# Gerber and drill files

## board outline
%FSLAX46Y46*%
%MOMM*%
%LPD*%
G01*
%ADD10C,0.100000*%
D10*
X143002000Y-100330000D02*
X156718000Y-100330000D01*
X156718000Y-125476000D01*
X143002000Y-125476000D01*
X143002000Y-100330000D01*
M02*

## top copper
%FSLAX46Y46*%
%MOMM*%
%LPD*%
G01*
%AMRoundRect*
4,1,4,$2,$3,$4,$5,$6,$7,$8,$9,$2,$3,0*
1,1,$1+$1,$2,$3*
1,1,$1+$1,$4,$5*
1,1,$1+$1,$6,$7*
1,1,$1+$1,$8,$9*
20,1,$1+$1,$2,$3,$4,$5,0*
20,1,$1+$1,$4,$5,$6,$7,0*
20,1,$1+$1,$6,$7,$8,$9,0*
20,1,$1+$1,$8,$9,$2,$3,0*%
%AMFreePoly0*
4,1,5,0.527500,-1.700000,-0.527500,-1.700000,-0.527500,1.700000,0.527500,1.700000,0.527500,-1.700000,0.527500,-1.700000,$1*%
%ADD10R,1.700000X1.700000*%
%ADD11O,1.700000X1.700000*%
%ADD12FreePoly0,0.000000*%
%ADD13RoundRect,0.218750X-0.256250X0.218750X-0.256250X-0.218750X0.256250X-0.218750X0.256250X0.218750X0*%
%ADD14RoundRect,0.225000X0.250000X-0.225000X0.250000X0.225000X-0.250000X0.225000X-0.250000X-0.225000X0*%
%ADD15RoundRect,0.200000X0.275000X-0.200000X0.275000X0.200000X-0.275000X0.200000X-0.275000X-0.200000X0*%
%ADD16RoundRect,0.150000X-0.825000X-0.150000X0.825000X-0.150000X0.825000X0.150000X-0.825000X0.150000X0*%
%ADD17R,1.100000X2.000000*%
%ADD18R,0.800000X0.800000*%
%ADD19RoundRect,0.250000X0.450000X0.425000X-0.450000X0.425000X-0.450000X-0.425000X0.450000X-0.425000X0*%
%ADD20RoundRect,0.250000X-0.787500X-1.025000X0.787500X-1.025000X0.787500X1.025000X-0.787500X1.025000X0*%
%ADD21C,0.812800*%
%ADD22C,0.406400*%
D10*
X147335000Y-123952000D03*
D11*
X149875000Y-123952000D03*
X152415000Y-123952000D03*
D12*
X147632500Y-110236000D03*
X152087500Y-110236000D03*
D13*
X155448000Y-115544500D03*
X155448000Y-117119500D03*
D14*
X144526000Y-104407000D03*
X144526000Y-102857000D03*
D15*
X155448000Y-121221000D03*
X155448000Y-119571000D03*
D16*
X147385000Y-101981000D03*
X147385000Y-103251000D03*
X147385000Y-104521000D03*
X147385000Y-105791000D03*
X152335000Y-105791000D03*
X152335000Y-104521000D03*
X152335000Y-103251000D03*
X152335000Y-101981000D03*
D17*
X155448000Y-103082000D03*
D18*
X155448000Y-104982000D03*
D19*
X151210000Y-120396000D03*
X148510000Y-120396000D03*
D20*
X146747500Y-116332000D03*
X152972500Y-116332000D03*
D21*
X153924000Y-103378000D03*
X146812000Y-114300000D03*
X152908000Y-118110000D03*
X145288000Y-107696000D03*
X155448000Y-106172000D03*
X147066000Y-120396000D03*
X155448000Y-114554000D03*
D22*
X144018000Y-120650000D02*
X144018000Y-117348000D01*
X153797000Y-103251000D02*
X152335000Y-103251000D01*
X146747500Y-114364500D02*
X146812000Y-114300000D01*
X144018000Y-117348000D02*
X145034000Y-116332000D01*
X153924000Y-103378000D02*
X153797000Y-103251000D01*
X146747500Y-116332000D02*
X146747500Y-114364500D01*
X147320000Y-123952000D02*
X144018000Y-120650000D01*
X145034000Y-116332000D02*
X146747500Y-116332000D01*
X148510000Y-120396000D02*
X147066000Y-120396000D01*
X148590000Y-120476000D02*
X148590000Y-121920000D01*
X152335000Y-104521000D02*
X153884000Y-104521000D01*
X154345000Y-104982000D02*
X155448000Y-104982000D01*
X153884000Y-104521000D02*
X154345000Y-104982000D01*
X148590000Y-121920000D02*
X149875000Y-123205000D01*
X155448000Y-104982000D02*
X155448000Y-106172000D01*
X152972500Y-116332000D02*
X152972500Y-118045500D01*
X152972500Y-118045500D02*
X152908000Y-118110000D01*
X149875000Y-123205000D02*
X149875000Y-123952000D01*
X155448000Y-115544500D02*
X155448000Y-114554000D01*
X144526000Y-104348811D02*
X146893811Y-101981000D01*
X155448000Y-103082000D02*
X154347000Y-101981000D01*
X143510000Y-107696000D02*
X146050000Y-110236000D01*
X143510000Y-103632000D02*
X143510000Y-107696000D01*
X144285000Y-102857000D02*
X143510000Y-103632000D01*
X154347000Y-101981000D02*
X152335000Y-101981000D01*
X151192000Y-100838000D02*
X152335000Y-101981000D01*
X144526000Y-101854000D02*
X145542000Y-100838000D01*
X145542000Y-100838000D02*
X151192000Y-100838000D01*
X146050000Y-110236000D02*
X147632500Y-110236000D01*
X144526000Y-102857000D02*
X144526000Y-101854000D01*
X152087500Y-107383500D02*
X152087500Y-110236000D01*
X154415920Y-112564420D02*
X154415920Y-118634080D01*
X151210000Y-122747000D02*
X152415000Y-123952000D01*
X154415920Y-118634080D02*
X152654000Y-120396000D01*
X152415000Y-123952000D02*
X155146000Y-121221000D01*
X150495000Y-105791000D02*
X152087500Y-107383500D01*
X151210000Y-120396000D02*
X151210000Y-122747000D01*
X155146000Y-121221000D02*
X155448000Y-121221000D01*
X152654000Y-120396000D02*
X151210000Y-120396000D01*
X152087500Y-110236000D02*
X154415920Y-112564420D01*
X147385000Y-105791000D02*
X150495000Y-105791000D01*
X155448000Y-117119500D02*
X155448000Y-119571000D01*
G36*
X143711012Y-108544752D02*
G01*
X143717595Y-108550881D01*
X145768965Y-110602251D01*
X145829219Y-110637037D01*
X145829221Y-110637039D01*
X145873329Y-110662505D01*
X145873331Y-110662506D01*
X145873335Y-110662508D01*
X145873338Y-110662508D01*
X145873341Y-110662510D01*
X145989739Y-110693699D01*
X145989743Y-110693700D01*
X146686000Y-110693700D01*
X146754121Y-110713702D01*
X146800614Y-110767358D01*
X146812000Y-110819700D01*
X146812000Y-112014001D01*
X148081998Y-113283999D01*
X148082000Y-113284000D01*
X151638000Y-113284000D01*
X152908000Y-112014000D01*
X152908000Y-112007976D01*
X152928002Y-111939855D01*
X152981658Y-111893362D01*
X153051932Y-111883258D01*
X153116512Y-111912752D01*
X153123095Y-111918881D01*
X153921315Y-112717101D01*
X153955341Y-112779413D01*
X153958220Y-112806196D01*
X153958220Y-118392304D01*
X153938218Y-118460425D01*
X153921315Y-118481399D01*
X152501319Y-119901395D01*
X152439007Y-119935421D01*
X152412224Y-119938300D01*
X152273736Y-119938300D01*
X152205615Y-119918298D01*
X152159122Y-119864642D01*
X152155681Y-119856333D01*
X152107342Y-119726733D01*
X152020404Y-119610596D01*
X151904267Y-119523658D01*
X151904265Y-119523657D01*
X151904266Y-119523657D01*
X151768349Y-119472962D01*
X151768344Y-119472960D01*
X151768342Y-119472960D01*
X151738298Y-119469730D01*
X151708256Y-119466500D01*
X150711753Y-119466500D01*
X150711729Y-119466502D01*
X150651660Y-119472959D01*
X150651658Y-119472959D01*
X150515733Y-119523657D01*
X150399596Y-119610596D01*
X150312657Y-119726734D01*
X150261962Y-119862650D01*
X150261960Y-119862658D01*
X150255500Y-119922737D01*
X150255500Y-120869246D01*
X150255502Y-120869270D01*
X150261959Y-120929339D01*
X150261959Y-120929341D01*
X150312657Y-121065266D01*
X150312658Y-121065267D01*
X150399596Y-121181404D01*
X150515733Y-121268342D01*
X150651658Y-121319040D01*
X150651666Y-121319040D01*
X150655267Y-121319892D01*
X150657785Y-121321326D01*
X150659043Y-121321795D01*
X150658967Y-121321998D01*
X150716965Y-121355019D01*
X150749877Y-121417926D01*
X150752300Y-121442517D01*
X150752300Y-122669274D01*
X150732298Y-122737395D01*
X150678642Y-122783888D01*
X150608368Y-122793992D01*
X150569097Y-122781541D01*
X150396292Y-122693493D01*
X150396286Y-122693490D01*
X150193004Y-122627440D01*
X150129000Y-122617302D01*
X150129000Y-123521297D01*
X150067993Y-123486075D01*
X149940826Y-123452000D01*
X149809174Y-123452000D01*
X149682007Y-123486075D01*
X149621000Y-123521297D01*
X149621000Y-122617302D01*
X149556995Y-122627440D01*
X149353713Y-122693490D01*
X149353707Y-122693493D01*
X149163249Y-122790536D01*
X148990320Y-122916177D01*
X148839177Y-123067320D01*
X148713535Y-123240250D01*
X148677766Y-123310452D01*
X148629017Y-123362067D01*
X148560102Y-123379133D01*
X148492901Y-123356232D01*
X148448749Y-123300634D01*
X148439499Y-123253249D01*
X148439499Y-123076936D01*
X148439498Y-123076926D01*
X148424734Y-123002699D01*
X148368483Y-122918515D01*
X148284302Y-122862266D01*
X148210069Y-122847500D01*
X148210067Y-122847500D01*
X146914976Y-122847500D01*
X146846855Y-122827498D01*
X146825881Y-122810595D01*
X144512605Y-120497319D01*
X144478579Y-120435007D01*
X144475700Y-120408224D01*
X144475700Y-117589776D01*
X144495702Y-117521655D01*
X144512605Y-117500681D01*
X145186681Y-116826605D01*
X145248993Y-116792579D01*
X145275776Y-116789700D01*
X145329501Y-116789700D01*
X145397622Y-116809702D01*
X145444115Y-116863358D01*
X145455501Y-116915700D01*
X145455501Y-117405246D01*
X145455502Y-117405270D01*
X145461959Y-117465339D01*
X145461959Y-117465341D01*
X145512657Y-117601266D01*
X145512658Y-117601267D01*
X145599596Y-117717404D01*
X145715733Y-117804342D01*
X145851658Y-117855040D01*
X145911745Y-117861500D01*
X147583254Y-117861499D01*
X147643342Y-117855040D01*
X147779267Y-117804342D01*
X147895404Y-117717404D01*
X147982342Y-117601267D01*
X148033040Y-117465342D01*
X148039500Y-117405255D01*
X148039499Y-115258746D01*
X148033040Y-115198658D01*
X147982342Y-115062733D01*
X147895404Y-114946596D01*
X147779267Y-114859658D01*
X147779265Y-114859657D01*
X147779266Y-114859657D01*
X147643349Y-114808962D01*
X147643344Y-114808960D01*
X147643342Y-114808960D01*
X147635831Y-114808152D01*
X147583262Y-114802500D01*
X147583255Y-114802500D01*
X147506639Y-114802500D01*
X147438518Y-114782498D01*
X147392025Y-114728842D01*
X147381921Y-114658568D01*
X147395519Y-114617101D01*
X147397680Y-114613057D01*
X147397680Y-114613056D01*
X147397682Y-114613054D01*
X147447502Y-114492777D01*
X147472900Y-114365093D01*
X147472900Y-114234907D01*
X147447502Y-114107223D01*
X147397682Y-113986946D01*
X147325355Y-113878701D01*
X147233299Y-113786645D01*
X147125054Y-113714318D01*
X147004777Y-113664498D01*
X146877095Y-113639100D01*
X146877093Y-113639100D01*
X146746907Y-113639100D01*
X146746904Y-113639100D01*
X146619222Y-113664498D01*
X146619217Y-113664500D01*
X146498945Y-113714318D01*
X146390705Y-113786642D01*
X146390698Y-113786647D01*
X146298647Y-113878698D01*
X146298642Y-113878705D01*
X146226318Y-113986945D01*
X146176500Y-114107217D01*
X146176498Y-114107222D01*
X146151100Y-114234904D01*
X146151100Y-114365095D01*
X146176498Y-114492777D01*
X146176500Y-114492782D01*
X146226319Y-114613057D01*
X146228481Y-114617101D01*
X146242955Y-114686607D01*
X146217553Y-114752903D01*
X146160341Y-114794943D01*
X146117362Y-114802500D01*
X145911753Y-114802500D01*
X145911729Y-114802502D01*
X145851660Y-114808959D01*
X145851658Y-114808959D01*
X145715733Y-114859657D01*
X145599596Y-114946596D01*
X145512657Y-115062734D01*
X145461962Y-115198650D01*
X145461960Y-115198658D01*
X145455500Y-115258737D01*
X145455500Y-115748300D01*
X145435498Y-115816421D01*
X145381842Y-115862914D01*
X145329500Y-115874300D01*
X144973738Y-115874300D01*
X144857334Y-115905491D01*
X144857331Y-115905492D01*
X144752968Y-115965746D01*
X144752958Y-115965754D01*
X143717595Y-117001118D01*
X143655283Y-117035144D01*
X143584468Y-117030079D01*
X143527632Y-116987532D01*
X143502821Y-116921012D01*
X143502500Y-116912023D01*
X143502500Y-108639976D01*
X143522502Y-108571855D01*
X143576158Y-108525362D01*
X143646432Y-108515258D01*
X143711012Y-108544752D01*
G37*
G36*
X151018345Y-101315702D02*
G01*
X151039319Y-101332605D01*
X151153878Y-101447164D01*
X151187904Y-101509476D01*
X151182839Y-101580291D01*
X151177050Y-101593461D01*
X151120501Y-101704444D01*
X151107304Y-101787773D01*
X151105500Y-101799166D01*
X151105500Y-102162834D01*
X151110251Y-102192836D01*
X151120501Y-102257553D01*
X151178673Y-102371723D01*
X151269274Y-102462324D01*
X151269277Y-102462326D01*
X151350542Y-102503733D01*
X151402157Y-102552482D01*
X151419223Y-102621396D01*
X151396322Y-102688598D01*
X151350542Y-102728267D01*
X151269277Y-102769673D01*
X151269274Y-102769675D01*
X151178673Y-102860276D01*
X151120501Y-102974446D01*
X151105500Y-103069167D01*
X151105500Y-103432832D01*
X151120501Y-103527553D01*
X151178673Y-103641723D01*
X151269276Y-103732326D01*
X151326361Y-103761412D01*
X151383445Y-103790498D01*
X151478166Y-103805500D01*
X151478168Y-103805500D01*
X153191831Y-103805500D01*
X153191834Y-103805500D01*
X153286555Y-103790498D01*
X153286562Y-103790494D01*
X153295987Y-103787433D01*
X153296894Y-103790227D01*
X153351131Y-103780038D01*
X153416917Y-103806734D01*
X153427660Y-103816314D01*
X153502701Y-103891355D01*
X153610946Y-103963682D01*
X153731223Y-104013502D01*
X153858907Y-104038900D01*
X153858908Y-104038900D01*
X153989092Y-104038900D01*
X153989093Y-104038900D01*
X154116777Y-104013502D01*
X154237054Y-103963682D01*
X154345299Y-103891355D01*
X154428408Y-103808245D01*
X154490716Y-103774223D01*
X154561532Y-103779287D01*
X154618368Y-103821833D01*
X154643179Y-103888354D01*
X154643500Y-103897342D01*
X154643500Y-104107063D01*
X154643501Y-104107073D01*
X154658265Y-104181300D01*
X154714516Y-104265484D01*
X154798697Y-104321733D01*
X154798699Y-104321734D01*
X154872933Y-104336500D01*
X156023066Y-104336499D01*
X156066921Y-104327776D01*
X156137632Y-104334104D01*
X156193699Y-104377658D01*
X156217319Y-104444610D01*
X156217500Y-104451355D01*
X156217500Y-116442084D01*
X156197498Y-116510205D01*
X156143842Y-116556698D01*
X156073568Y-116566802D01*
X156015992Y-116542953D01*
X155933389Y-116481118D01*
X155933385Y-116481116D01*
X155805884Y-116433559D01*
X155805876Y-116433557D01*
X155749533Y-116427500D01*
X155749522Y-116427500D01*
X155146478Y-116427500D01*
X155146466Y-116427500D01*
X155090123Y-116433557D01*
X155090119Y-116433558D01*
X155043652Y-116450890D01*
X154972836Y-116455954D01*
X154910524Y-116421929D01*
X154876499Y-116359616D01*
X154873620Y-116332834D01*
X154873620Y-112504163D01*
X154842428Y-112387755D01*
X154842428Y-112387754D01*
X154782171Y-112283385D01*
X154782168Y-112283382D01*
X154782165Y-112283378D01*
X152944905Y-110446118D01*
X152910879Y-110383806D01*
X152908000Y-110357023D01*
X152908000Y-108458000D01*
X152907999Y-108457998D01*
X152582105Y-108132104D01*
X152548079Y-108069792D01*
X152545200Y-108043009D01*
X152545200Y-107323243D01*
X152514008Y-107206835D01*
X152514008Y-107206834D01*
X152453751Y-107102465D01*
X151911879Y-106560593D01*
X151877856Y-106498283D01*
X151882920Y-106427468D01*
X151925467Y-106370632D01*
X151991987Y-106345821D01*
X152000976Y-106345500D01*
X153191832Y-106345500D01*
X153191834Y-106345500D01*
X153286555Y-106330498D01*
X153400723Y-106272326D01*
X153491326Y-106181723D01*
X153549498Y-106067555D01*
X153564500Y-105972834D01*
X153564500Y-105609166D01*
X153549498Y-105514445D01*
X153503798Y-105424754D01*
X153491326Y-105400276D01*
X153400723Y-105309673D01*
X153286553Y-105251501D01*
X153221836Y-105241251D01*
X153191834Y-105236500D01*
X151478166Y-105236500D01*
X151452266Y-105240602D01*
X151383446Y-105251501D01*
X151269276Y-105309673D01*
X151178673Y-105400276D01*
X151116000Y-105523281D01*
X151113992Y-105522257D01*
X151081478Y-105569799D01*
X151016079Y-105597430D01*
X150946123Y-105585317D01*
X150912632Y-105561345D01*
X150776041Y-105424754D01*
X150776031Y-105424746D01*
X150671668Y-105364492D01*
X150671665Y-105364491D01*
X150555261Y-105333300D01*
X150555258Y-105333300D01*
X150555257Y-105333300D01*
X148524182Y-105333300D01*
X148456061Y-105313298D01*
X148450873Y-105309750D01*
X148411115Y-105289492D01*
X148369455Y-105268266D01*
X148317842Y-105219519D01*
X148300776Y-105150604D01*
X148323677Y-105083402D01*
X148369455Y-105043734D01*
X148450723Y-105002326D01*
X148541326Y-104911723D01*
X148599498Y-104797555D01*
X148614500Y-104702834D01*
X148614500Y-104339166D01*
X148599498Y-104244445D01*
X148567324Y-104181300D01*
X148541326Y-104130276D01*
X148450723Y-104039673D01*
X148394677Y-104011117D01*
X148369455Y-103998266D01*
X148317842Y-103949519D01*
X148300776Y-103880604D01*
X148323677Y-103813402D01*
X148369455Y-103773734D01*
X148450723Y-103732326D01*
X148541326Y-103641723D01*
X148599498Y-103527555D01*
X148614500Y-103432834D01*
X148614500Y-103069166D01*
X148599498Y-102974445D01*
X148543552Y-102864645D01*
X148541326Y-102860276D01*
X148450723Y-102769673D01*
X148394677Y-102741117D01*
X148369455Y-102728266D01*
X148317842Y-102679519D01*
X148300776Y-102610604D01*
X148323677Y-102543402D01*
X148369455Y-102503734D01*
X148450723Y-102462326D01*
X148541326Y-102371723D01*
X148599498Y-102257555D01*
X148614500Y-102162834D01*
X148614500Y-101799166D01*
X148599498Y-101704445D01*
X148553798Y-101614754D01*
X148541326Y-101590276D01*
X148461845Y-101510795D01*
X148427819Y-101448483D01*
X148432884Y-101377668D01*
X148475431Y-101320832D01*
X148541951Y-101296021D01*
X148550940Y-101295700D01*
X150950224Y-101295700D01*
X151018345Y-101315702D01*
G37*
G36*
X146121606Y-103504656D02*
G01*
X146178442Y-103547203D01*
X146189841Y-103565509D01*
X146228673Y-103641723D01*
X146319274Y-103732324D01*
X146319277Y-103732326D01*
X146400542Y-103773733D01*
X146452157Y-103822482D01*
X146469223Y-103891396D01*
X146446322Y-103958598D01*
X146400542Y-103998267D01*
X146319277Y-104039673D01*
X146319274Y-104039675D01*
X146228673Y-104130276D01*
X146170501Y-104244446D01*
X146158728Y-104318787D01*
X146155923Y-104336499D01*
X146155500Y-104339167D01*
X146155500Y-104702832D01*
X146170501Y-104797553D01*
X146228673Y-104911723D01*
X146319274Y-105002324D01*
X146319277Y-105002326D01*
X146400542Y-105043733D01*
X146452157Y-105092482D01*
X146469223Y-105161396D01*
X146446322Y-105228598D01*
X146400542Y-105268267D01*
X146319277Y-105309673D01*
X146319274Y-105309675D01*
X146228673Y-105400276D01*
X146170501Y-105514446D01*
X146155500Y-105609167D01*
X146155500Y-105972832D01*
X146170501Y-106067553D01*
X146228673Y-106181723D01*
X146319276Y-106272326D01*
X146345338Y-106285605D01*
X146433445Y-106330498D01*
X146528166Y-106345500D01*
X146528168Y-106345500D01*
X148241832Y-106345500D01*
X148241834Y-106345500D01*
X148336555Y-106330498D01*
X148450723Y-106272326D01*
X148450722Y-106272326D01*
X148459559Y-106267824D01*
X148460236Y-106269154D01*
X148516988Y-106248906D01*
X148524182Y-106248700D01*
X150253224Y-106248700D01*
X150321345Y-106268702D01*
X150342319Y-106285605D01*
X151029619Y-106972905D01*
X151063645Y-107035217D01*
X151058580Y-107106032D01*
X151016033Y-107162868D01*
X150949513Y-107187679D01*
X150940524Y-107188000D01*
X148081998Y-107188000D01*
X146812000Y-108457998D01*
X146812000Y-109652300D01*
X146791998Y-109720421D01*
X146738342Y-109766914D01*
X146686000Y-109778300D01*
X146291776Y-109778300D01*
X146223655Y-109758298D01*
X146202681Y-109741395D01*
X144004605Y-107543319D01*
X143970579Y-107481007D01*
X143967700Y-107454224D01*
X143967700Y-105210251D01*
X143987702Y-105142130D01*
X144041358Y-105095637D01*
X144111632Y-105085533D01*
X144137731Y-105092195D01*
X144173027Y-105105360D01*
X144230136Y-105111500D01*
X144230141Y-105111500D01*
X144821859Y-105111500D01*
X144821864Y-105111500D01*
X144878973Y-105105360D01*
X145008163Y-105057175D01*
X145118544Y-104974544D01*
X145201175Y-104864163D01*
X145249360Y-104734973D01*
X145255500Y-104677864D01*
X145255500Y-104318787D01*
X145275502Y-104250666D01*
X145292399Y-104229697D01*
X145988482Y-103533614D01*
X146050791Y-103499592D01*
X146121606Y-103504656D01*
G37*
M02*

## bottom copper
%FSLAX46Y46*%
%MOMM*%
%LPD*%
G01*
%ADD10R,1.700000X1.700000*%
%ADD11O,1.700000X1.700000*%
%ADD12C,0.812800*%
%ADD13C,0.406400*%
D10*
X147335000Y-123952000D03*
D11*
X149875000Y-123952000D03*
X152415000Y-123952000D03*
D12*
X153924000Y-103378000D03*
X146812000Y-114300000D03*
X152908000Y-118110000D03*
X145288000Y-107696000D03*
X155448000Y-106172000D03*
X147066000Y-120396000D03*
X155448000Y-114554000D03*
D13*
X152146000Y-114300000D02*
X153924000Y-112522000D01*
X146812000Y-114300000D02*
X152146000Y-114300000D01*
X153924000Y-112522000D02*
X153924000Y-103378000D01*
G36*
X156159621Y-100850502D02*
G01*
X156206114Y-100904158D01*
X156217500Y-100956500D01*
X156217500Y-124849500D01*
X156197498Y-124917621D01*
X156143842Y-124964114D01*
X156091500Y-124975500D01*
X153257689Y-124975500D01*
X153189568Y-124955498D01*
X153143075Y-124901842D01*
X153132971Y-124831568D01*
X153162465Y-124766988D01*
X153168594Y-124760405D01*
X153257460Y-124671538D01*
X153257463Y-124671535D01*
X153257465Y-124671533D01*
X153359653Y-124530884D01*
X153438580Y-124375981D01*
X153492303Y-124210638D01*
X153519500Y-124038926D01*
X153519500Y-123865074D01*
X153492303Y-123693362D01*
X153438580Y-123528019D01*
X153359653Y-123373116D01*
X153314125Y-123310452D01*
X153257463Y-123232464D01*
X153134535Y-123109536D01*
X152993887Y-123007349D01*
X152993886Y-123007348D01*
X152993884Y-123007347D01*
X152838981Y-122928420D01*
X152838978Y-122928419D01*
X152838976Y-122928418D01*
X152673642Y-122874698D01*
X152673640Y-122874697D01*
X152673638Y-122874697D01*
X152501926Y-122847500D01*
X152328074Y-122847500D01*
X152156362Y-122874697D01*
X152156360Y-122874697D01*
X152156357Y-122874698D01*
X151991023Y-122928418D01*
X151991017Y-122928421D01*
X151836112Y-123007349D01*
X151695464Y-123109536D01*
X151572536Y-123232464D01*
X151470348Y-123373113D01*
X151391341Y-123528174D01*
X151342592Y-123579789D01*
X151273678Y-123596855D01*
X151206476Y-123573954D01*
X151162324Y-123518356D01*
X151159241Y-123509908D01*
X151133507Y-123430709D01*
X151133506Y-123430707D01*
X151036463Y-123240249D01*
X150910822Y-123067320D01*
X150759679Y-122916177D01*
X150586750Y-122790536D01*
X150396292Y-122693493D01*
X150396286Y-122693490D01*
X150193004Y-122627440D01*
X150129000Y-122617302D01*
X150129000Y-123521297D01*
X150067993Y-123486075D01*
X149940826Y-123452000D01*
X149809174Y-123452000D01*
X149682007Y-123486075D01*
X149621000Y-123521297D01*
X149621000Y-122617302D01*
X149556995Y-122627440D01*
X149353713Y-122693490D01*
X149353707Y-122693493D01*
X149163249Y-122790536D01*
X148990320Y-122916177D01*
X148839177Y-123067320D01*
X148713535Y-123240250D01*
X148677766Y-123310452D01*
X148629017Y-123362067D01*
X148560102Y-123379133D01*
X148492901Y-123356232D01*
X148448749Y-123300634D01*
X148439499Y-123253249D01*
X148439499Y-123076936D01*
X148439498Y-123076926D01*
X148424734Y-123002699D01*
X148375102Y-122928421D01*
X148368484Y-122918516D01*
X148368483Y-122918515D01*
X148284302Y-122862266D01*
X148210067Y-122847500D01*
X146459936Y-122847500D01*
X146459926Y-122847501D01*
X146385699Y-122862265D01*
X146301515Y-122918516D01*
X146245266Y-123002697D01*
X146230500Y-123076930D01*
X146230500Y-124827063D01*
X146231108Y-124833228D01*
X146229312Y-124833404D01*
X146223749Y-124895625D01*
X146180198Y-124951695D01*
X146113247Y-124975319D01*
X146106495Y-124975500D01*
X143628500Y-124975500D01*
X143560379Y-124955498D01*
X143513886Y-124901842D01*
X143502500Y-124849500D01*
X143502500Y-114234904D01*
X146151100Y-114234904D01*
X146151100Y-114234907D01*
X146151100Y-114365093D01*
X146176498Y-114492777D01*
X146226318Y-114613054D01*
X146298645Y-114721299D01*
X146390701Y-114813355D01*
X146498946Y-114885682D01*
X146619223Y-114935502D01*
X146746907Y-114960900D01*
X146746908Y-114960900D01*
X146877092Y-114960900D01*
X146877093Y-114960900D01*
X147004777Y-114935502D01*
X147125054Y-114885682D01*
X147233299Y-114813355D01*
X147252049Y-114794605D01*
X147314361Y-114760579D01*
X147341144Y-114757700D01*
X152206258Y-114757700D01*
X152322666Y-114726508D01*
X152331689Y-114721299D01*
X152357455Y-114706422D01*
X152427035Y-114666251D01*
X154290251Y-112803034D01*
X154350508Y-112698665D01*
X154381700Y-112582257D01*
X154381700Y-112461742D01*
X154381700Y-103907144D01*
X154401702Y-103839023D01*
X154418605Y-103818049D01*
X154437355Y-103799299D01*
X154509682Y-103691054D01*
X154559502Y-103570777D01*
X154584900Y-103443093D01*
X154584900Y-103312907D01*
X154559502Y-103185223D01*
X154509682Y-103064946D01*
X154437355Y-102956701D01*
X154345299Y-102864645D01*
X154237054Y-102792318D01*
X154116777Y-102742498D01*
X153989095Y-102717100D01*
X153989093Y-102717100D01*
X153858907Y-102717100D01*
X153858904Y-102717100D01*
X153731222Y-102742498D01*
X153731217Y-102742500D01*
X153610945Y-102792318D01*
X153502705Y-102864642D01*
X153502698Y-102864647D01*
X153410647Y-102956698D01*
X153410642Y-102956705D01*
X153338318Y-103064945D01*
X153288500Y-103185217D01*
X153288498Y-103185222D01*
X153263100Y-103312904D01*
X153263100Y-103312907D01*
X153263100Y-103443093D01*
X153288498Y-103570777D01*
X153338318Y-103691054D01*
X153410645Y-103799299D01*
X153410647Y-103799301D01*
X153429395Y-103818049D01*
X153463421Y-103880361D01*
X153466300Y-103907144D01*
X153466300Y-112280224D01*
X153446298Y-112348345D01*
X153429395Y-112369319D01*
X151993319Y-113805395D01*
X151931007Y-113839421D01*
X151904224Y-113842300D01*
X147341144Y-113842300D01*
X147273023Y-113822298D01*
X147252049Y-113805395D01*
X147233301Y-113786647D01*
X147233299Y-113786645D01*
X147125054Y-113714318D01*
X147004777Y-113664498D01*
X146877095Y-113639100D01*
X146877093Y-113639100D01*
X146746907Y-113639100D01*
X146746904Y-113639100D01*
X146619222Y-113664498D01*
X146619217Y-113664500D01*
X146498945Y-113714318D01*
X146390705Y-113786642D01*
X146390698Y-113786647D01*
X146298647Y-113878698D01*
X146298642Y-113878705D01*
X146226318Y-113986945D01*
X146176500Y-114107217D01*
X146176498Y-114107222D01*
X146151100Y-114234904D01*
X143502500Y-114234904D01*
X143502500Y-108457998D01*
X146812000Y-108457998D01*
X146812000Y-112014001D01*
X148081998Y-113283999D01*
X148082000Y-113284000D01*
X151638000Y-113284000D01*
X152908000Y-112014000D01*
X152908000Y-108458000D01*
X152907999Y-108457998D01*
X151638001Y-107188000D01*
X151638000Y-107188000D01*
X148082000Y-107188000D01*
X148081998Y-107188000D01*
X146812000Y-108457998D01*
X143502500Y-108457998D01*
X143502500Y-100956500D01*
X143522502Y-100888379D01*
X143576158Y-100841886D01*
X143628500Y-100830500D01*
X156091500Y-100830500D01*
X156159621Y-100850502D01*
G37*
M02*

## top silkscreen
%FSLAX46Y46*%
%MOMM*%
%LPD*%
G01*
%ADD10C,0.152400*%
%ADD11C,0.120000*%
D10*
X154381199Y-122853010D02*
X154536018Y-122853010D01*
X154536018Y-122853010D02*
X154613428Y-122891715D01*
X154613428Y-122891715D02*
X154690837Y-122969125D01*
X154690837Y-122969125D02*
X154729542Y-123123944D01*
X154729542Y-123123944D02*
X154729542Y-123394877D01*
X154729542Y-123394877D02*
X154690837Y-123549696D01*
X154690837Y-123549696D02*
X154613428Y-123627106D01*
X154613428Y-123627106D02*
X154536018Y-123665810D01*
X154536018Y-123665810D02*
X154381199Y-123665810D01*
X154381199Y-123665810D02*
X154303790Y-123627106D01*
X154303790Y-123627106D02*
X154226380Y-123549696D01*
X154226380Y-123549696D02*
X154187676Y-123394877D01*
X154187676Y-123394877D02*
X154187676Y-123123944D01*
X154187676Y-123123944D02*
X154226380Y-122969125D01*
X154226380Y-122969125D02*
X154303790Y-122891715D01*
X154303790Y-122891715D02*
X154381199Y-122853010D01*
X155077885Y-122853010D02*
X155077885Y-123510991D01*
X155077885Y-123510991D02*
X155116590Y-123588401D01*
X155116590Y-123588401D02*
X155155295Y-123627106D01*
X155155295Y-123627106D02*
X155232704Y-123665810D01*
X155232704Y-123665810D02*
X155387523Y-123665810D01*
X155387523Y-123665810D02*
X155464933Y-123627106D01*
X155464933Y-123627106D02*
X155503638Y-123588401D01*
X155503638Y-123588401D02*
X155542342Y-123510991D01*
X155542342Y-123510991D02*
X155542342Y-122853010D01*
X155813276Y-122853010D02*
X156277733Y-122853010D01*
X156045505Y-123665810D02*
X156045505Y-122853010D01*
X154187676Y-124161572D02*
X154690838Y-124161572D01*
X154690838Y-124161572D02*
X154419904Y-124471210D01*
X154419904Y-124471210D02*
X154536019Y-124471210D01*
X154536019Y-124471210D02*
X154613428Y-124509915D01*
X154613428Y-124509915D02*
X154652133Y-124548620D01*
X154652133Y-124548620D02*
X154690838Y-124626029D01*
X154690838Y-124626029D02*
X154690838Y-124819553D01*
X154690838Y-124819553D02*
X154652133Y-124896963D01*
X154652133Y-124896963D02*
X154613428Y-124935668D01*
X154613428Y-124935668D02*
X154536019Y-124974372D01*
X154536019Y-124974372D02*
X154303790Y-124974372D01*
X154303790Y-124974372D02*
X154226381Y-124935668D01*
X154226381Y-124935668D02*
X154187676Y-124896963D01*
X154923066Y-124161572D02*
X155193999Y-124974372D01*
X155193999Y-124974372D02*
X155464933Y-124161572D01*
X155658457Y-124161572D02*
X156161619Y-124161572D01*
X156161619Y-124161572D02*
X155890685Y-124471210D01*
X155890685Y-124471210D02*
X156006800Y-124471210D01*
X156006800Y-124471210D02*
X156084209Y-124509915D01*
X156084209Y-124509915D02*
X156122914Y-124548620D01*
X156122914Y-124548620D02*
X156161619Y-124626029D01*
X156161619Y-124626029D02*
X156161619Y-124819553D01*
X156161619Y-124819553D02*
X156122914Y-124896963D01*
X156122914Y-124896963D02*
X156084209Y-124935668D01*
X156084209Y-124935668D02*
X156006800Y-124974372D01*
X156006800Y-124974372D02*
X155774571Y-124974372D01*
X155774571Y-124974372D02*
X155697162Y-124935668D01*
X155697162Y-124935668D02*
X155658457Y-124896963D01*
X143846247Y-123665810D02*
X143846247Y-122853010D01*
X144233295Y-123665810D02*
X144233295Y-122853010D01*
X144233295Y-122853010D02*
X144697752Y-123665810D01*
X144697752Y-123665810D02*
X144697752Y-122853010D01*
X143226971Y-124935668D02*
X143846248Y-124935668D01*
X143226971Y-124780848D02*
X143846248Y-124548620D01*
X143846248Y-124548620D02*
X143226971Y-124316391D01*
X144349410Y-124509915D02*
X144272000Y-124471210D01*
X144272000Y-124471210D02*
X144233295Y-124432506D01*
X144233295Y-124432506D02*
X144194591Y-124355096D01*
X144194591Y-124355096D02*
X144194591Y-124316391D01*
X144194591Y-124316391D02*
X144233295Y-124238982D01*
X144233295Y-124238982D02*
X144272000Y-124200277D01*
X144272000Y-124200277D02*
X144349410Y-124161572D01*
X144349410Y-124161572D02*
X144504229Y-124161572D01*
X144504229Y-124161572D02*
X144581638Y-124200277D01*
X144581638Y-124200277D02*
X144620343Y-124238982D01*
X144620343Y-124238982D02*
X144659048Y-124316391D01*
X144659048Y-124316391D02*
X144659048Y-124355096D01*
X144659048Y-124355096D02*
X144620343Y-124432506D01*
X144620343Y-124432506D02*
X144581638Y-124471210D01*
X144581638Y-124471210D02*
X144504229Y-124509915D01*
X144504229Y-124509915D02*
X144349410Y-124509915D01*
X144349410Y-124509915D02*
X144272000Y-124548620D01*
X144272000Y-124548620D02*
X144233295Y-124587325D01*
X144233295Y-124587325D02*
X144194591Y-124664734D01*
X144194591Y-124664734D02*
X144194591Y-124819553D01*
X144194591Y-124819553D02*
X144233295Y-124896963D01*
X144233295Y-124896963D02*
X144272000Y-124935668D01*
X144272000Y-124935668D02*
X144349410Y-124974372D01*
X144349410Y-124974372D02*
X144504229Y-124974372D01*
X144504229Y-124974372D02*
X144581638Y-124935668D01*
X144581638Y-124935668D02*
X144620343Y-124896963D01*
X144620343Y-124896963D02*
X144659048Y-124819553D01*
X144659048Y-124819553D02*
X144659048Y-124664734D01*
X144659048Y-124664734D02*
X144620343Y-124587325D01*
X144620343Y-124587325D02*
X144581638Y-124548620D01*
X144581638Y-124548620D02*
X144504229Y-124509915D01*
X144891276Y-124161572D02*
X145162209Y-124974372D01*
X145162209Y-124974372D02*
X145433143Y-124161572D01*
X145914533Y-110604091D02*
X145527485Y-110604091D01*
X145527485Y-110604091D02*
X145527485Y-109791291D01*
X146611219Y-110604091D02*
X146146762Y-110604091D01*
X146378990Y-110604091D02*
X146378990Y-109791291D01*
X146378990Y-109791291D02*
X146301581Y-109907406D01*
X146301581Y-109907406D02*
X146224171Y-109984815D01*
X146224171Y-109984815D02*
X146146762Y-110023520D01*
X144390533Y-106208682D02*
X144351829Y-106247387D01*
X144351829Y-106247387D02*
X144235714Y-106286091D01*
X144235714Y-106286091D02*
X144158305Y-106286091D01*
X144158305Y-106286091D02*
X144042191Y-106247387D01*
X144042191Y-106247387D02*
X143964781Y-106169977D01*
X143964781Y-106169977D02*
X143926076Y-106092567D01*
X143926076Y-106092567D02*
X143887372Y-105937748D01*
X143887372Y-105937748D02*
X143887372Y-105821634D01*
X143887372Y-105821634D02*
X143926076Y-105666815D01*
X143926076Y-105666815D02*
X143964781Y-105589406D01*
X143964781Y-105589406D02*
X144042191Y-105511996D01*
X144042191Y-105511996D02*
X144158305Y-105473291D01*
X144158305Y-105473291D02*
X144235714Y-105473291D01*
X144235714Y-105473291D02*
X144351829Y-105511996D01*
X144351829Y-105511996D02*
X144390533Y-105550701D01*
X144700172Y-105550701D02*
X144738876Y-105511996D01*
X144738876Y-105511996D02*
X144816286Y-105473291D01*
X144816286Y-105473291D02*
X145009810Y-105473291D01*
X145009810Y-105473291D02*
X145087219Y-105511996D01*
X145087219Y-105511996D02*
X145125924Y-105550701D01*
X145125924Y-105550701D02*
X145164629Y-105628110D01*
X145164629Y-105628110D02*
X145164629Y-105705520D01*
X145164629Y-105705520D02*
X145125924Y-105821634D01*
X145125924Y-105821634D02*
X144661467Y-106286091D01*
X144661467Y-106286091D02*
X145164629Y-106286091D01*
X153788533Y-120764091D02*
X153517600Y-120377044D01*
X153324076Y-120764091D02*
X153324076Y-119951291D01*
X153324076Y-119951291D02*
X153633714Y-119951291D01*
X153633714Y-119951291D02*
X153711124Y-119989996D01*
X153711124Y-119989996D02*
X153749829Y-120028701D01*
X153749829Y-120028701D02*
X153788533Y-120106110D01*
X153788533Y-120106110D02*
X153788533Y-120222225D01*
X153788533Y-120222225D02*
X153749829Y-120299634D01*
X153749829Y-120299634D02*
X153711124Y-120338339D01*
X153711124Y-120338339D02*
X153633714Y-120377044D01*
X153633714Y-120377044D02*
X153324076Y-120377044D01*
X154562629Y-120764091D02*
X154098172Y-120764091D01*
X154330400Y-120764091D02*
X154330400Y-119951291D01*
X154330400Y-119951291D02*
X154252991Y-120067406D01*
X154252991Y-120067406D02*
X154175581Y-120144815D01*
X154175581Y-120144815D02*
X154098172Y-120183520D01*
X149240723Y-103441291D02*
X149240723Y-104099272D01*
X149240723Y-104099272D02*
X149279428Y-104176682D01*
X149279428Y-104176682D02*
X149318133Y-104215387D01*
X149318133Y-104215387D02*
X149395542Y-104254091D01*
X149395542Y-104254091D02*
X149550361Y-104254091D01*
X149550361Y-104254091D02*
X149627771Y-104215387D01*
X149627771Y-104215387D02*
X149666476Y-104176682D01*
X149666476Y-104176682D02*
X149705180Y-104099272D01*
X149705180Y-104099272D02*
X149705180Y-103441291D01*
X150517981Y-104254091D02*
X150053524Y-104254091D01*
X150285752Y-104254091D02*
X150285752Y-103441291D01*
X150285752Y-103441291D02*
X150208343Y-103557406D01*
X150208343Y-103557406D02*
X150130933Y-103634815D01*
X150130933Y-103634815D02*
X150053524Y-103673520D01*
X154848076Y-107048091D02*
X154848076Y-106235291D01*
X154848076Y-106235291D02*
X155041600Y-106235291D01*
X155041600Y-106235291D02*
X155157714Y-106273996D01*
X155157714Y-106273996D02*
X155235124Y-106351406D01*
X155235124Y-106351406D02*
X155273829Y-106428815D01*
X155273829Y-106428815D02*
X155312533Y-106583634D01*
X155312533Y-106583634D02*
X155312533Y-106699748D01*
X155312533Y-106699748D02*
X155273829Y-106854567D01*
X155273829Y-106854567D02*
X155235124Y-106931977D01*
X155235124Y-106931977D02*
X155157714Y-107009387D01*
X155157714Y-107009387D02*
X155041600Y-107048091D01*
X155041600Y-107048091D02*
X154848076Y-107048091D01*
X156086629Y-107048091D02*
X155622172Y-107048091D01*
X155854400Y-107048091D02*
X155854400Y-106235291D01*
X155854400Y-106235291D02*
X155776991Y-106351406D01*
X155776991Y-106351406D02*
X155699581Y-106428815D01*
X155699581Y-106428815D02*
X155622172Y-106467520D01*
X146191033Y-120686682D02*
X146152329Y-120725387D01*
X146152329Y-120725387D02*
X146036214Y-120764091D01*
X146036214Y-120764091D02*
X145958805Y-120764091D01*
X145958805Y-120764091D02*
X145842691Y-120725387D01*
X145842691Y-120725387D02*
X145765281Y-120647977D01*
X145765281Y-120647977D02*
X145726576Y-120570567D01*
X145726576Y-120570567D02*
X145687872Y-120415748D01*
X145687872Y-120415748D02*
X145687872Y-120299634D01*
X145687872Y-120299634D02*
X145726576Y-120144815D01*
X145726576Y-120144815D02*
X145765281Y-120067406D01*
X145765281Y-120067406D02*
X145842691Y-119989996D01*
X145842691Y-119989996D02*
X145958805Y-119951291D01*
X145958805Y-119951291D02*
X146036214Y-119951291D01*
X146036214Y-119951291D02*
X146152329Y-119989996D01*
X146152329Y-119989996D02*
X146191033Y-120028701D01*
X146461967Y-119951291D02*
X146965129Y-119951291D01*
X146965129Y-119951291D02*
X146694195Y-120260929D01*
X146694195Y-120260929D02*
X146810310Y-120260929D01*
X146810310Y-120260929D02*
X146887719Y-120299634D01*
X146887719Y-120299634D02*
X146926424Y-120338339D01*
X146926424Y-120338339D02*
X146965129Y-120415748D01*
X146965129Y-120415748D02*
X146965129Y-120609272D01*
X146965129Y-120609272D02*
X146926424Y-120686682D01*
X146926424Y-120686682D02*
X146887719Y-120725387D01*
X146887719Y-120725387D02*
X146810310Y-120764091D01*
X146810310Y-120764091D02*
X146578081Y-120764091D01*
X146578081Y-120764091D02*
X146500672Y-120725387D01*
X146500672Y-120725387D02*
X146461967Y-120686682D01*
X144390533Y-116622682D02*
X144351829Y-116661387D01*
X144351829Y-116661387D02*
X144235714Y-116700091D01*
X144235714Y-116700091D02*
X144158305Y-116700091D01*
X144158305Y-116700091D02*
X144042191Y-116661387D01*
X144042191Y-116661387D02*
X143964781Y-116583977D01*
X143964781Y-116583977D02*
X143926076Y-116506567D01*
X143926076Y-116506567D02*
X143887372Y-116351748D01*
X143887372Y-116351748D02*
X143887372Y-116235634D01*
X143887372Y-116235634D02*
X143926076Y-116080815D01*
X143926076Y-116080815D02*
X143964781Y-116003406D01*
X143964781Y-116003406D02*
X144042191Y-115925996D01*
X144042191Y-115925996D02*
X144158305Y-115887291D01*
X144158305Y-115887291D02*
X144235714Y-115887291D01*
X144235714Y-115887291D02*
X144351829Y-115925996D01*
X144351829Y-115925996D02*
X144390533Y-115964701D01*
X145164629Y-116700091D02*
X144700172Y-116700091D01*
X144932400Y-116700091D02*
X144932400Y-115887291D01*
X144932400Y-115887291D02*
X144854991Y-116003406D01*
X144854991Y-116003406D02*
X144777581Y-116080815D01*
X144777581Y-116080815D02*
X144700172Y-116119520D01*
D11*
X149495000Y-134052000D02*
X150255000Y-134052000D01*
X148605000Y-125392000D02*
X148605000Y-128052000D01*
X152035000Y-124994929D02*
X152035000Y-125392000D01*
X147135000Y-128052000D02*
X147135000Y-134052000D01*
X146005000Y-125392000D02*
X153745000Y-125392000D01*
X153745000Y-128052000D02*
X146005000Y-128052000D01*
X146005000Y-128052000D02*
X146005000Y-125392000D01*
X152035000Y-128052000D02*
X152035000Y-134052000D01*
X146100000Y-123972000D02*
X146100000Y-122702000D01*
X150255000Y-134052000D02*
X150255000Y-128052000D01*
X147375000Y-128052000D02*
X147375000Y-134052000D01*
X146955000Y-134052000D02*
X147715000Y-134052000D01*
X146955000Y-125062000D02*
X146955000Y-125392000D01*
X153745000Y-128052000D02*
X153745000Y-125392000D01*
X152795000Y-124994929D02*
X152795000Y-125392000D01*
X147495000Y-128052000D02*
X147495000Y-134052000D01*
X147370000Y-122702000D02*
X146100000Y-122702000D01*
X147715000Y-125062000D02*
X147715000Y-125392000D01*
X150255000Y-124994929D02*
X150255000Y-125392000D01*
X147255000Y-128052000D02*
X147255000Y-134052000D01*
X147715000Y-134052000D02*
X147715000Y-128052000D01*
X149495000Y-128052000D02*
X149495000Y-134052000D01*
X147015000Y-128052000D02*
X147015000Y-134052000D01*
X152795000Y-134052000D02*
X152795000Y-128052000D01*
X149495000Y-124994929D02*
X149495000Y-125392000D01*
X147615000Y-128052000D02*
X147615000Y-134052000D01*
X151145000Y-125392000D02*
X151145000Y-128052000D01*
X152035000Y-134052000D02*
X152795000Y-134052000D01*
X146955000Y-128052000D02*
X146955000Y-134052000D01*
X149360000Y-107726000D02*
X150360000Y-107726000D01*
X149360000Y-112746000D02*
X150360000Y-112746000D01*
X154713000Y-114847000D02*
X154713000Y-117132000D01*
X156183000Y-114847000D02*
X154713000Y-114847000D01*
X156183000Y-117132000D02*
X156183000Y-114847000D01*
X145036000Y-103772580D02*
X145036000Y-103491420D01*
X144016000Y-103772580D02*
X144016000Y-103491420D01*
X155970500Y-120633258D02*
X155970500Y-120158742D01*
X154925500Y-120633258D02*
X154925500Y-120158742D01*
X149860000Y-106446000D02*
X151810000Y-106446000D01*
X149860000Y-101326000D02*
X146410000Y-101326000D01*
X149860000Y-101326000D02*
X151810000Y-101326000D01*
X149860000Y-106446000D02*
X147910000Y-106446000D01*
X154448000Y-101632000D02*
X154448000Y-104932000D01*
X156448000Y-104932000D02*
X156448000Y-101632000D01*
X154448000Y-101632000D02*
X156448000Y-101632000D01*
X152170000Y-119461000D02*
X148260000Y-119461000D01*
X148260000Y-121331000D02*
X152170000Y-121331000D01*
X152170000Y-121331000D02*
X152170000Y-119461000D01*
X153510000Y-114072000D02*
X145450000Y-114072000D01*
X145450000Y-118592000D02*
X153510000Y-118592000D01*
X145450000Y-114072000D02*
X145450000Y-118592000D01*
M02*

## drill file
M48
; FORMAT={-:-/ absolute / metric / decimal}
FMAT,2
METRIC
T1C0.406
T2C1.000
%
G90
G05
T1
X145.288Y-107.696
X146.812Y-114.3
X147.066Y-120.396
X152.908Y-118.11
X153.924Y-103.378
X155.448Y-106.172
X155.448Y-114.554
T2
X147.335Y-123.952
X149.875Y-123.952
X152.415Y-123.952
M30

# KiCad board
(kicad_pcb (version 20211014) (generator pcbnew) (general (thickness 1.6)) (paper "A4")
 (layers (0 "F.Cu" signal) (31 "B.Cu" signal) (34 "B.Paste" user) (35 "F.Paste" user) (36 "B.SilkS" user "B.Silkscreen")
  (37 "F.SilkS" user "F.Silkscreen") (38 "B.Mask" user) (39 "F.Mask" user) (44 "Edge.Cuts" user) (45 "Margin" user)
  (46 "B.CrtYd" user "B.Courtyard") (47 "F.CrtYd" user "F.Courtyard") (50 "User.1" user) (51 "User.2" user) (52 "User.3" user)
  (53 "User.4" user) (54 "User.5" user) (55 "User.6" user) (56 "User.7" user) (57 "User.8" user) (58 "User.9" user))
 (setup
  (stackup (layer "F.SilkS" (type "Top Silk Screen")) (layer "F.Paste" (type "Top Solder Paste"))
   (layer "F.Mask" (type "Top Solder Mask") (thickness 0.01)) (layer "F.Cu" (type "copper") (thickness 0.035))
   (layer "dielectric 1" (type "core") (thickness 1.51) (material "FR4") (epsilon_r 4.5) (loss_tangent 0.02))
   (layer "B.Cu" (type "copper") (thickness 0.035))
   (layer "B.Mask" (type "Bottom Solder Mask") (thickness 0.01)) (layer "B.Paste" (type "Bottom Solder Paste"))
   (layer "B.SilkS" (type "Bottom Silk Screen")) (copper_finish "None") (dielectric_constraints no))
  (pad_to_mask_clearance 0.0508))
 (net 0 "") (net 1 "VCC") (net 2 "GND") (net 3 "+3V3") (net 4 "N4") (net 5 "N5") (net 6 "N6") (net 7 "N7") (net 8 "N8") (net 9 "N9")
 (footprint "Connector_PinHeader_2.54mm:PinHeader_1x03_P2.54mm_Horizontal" (layer "F.Cu") (at 147.335 123.952 90)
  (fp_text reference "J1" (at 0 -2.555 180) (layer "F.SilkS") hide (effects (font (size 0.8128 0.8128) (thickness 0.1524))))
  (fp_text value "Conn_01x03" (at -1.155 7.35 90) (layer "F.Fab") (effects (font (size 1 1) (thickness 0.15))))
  (fp_line (start -10.1 2.16) (end -10.1 2.92) (layer "F.SilkS") (width 0.12))
  (fp_line (start -1.44 1.27) (end -4.1 1.27) (layer "F.SilkS") (width 0.12))
  (fp_line (start -1.042929 4.7) (end -1.44 4.7) (layer "F.SilkS") (width 0.12))
  (fp_line (start -4.1 -0.2) (end -10.1 -0.2) (layer "F.SilkS") (width 0.12))
  (fp_line (start -1.44 -1.33) (end -1.44 6.41) (layer "F.SilkS") (width 0.12))
  (fp_line (start -4.1 6.41) (end -4.1 -1.33) (layer "F.SilkS") (width 0.12))
  (fp_line (start -4.1 -1.33) (end -1.44 -1.33) (layer "F.SilkS") (width 0.12))
  (fp_line (start -4.1 4.7) (end -10.1 4.7) (layer "F.SilkS") (width 0.12))
  (fp_line (start -0.02 -1.235) (end 1.25 -1.235) (layer "F.SilkS") (width 0.12))
  (fp_line (start -10.1 2.92) (end -4.1 2.92) (layer "F.SilkS") (width 0.12))
  (fp_line (start -4.1 0.04) (end -10.1 0.04) (layer "F.SilkS") (width 0.12))
  (fp_line (start -10.1 -0.38) (end -10.1 0.38) (layer "F.SilkS") (width 0.12))
  (fp_line (start -1.11 -0.38) (end -1.44 -0.38) (layer "F.SilkS") (width 0.12))
  (fp_line (start -4.1 6.41) (end -1.44 6.41) (layer "F.SilkS") (width 0.12))
  (fp_line (start -1.042929 5.46) (end -1.44 5.46) (layer "F.SilkS") (width 0.12))
  (fp_line (start -4.1 0.16) (end -10.1 0.16) (layer "F.SilkS") (width 0.12))
  (fp_line (start 1.25 0.035) (end 1.25 -1.235) (layer "F.SilkS") (width 0.12))
  (fp_line (start -1.11 0.38) (end -1.44 0.38) (layer "F.SilkS") (width 0.12))
  (fp_line (start -1.042929 2.92) (end -1.44 2.92) (layer "F.SilkS") (width 0.12))
  (fp_line (start -4.1 -0.08) (end -10.1 -0.08) (layer "F.SilkS") (width 0.12))
  (fp_line (start -10.1 0.38) (end -4.1 0.38) (layer "F.SilkS") (width 0.12))
  (fp_line (start -4.1 2.16) (end -10.1 2.16) (layer "F.SilkS") (width 0.12))
  (fp_line (start -4.1 -0.32) (end -10.1 -0.32) (layer "F.SilkS") (width 0.12))
  (fp_line (start -10.1 5.46) (end -4.1 5.46) (layer "F.SilkS") (width 0.12))
  (fp_line (start -1.042929 2.16) (end -1.44 2.16) (layer "F.SilkS") (width 0.12))
  (fp_line (start -4.1 0.28) (end -10.1 0.28) (layer "F.SilkS") (width 0.12))
  (fp_line (start -1.44 3.81) (end -4.1 3.81) (layer "F.SilkS") (width 0.12))
  (fp_line (start -10.1 4.7) (end -10.1 5.46) (layer "F.SilkS") (width 0.12))
  (fp_line (start -4.1 -0.38) (end -10.1 -0.38) (layer "F.SilkS") (width 0.12))
  (pad "1" thru_hole rect (at 0 0 90) (size 1.7 1.7) (drill 1) (layers *.Cu *.Mask) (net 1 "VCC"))
  (pad "2" thru_hole oval (at 0 2.54 90) (size 1.7 1.7) (drill 1) (layers *.Cu *.Mask) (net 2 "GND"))
  (pad "3" thru_hole oval (at 0 5.08 90) (size 1.7 1.7) (drill 1) (layers *.Cu *.Mask) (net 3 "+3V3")))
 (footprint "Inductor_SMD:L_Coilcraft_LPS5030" (layer "F.Cu") (at 149.86 110.236)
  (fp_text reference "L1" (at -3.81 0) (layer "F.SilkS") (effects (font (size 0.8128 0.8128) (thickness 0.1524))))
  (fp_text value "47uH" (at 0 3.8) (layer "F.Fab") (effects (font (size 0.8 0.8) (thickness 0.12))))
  (fp_line (start -0.5 -2.51) (end 0.5 -2.51) (layer "F.SilkS") (width 0.12))
  (fp_line (start -0.5 2.51) (end 0.5 2.51) (layer "F.SilkS") (width 0.12))
  (pad "1" smd custom locked (at -2.2275 0) (size 1.055 3.4) (layers "F.Cu" "F.Paste" "F.Mask") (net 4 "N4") (zone_connect 2)
   (options (clearance outline) (anchor rect)) (primitives))
  (pad "2" smd custom locked (at 2.2275 0) (size 1.055 3.4) (layers "F.Cu" "F.Paste" "F.Mask") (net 3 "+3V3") (zone_connect 2)
   (options (clearance outline) (anchor rect)) (primitives)))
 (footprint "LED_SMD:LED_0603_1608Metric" (layer "F.Cu") (at 155.448 116.332 -90)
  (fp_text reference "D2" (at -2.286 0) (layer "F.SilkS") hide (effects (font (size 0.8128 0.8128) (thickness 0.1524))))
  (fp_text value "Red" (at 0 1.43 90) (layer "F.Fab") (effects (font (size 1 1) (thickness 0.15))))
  (fp_line (start -1.485 0.735) (end 0.8 0.735) (layer "F.SilkS") (width 0.12))
  (fp_line (start -1.485 -0.735) (end -1.485 0.735) (layer "F.SilkS") (width 0.12))
  (fp_line (start 0.8 -0.735) (end -1.485 -0.735) (layer "F.SilkS") (width 0.12))
  (pad "1" smd roundrect locked (at -0.7875 0 270) (size 0.875 0.95) (layers "F.Cu" "F.Paste" "F.Mask") (roundrect_rratio 0.25)
   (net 2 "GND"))
  (pad "2" smd roundrect locked (at 0.7875 0 270) (size 0.875 0.95) (layers "F.Cu" "F.Paste" "F.Mask") (roundrect_rratio 0.25) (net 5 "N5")))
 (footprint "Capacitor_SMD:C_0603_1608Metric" (layer "F.Cu") (at 144.526 103.632 90)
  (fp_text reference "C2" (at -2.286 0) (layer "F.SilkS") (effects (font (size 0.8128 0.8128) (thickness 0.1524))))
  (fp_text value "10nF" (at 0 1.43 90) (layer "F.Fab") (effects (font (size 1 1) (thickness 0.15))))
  (fp_line (start -0.14058 0.51) (end 0.14058 0.51) (layer "F.SilkS") (width 0.12))
  (fp_line (start -0.14058 -0.51) (end 0.14058 -0.51) (layer "F.SilkS") (width 0.12))
  (pad "1" smd roundrect locked (at -0.775 0 90) (size 0.9 0.95) (layers "F.Cu" "F.Paste" "F.Mask") (roundrect_rratio 0.25) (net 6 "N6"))
  (pad "2" smd roundrect locked (at 0.775 0 90) (size 0.9 0.95) (layers "F.Cu" "F.Paste" "F.Mask") (roundrect_rratio 0.25) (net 4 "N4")))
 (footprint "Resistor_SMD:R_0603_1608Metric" (layer "F.Cu") (at 155.448 120.396 90)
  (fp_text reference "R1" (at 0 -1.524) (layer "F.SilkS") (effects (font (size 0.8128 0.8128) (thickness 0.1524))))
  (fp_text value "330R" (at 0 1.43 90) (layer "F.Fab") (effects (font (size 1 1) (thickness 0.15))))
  (fp_line (start -0.237258 0.5225) (end 0.237258 0.5225) (layer "F.SilkS") (width 0.12))
  (fp_line (start -0.237258 -0.5225) (end 0.237258 -0.5225) (layer "F.SilkS") (width 0.12))
  (pad "1" smd roundrect locked (at -0.825 0 90) (size 0.8 0.95) (layers "F.Cu" "F.Paste" "F.Mask") (roundrect_rratio 0.25) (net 3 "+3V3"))
  (pad "2" smd roundrect locked (at 0.825 0 90) (size 0.8 0.95) (layers "F.Cu" "F.Paste" "F.Mask") (roundrect_rratio 0.25) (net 5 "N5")))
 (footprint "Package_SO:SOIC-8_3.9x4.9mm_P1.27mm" (layer "F.Cu") (at 149.86 103.886)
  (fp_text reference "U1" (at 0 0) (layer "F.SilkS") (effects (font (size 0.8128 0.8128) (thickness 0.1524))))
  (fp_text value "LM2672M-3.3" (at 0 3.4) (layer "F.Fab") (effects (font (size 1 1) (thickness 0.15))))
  (fp_line (start 0 2.56) (end 1.95 2.56) (layer "F.SilkS") (width 0.12))
  (fp_line (start 0 -2.56) (end -3.45 -2.56) (layer "F.SilkS") (width 0.12))
  (fp_line (start 0 -2.56) (end 1.95 -2.56) (layer "F.SilkS") (width 0.12))
  (fp_line (start 0 2.56) (end -1.95 2.56) (layer "F.SilkS") (width 0.12))
  (pad "1" smd roundrect locked (at -2.475 -1.905) (size 1.95 0.6) (layers "F.Cu" "F.Paste" "F.Mask") (roundrect_rratio 0.25) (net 6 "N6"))
  (pad "2" smd roundrect locked (at -2.475 -0.635) (size 1.95 0.6) (layers "F.Cu" "F.Paste" "F.Mask") (roundrect_rratio 0.25) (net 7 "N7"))
  (pad "3" smd roundrect locked (at -2.475 0.635) (size 1.95 0.6) (layers "F.Cu" "F.Paste" "F.Mask") (roundrect_rratio 0.25) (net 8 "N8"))
  (pad "4" smd roundrect locked (at -2.475 1.905) (size 1.95 0.6) (layers "F.Cu" "F.Paste" "F.Mask") (roundrect_rratio 0.25) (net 3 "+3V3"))
  (pad "5" smd roundrect locked (at 2.475 1.905) (size 1.95 0.6) (layers "F.Cu" "F.Paste" "F.Mask") (roundrect_rratio 0.25) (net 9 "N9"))
  (pad "6" smd roundrect locked (at 2.475 0.635) (size 1.95 0.6) (layers "F.Cu" "F.Paste" "F.Mask") (roundrect_rratio 0.25) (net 2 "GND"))
  (pad "7" smd roundrect locked (at 2.475 -0.635) (size 1.95 0.6) (layers "F.Cu" "F.Paste" "F.Mask") (roundrect_rratio 0.25) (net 1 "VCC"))
  (pad "8" smd roundrect locked (at 2.475 -1.905) (size 1.95 0.6) (layers "F.Cu" "F.Paste" "F.Mask") (roundrect_rratio 0.25) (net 4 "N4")))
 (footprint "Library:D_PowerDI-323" (layer "F.Cu") (at 155.448 103.632 -90)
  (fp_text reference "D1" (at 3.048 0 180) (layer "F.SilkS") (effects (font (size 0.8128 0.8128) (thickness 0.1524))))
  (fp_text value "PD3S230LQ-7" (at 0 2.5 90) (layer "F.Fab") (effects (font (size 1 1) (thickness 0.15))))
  (fp_line (start -2 1) (end 1.3 1) (layer "F.SilkS") (width 0.12))
  (fp_line (start 1.3 -1) (end -2 -1) (layer "F.SilkS") (width 0.12))
  (fp_line (start -2 1) (end -2 -1) (layer "F.SilkS") (width 0.12))
  (pad "1" smd rect (at -0.55 0 90) (size 2 1.1) (layers "F.Cu" "F.Paste" "F.Mask") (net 4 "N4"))
  (pad "2" smd rect (at 1.35 0 90) (size 0.8 0.8) (layers "F.Cu" "F.Paste" "F.Mask") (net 2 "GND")))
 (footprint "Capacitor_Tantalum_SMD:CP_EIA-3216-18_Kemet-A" (layer "F.Cu") (at 149.86 120.396 180)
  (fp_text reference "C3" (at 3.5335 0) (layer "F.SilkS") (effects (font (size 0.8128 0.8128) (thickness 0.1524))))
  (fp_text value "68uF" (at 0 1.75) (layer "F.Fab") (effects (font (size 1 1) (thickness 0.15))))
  (fp_line (start -2.31 0.935) (end 1.6 0.935) (layer "F.SilkS") (width 0.12))
  (fp_line (start 1.6 -0.935) (end -2.31 -0.935) (layer "F.SilkS") (width 0.12))
  (fp_line (start -2.31 -0.935) (end -2.31 0.935) (layer "F.SilkS") (width 0.12))
  (pad "1" smd roundrect locked (at -1.35 0 180) (size 1.4 1.35) (layers "F.Cu" "F.Paste" "F.Mask") (roundrect_rratio 0.1851851852)
   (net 3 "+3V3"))
  (pad "2" smd roundrect locked (at 1.35 0 180) (size 1.4 1.35) (layers "F.Cu" "F.Paste" "F.Mask") (roundrect_rratio 0.1851851852)
   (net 2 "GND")))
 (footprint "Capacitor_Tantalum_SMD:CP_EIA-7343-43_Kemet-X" (layer "F.Cu") (at 149.86 116.332)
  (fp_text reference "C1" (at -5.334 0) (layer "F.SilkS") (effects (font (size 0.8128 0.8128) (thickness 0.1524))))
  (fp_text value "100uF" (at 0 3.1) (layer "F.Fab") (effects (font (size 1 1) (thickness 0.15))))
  (fp_line (start 3.65 -2.26) (end -4.41 -2.26) (layer "F.SilkS") (width 0.12))
  (fp_line (start -4.41 2.26) (end 3.65 2.26) (layer "F.SilkS") (width 0.12))
  (fp_line (start -4.41 -2.26) (end -4.41 2.26) (layer "F.SilkS") (width 0.12))
  (pad "1" smd roundrect locked (at -3.1125 0) (size 2.075 2.55) (layers "F.Cu" "F.Paste" "F.Mask") (roundrect_rratio 0.1204819277)
   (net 1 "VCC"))
  (pad "2" smd roundrect locked (at 3.1125 0) (size 2.075 2.55) (layers "F.Cu" "F.Paste" "F.Mask") (roundrect_rratio 0.1204819277)
   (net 2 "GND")))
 (gr_rect (start 143.002 100.33) (end 156.718 125.476) (layer "Edge.Cuts") (width 0.1) (fill none))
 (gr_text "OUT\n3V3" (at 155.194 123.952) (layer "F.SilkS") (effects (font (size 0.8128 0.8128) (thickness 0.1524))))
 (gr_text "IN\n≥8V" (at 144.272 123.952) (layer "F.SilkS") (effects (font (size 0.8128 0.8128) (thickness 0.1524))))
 (segment (start 144.018 120.65) (end 144.018 117.348) (width 0.4064) (layer "F.Cu") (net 1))
 (segment (start 153.797 103.251) (end 152.335 103.251) (width 0.4064) (layer "F.Cu") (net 1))
 (segment (start 146.7475 114.3645) (end 146.812 114.3) (width 0.4064) (layer "F.Cu") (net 1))
 (segment (start 144.018 117.348) (end 145.034 116.332) (width 0.4064) (layer "F.Cu") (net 1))
 (segment (start 153.924 103.378) (end 153.797 103.251) (width 0.4064) (layer "F.Cu") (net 1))
 (segment (start 146.7475 116.332) (end 146.7475 114.3645) (width 0.4064) (layer "F.Cu") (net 1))
 (segment (start 147.32 123.952) (end 144.018 120.65) (width 0.4064) (layer "F.Cu") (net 1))
 (segment (start 145.034 116.332) (end 146.7475 116.332) (width 0.4064) (layer "F.Cu") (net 1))
 (via (at 153.924 103.378) (size 0.8128) (drill 0.4064) (layers "F.Cu" "B.Cu") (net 1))
 (via (at 146.812 114.3) (size 0.8128) (drill 0.4064) (layers "F.Cu" "B.Cu") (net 1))
 (segment (start 152.146 114.3) (end 153.924 112.522) (width 0.4064) (layer "B.Cu") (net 1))
 (segment (start 146.812 114.3) (end 152.146 114.3) (width 0.4064) (layer "B.Cu") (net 1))
 (segment (start 153.924 112.522) (end 153.924 103.378) (width 0.4064) (layer "B.Cu") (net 1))
 (segment (start 148.51 120.396) (end 147.066 120.396) (width 0.4064) (layer "F.Cu") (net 2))
 (segment (start 148.59 120.476) (end 148.59 121.92) (width 0.4064) (layer "F.Cu") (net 2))
 (segment (start 152.335 104.521) (end 153.884 104.521) (width 0.4064) (layer "F.Cu") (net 2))
 (segment (start 154.345 104.982) (end 155.448 104.982) (width 0.4064) (layer "F.Cu") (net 2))
 (segment (start 153.884 104.521) (end 154.345 104.982) (width 0.4064) (layer "F.Cu") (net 2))
 (segment (start 148.59 121.92) (end 149.875 123.205) (width 0.4064) (layer "F.Cu") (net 2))
 (segment (start 155.448 104.982) (end 155.448 106.172) (width 0.4064) (layer "F.Cu") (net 2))
 (segment (start 152.9725 116.332) (end 152.9725 118.0455) (width 0.4064) (layer "F.Cu") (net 2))
 (segment (start 152.9725 118.0455) (end 152.908 118.11) (width 0.4064) (layer "F.Cu") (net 2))
 (segment (start 149.875 123.205) (end 149.875 123.952) (width 0.4064) (layer "F.Cu") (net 2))
 (segment (start 155.448 115.5445) (end 155.448 114.554) (width 0.4064) (layer "F.Cu") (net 2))
 (via (at 152.908 118.11) (size 0.8128) (drill 0.4064) (layers "F.Cu" "B.Cu") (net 2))
 (via (at 145.288 107.696) (size 0.8128) (drill 0.4064) (layers "F.Cu" "B.Cu") (free) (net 2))
 (via (at 155.448 106.172) (size 0.8128) (drill 0.4064) (layers "F.Cu" "B.Cu") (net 2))
 (via (at 147.066 120.396) (size 0.8128) (drill 0.4064) (layers "F.Cu" "B.Cu") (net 2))
 (via (at 155.448 114.554) (size 0.8128) (drill 0.4064) (layers "F.Cu" "B.Cu") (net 2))
 (segment (start 144.526 104.348811) (end 146.893811 101.981) (width 0.4064) (layer "F.Cu") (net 6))
 (segment (start 155.448 103.082) (end 154.347 101.981) (width 0.4064) (layer "F.Cu") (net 4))
 (segment (start 143.51 107.696) (end 146.05 110.236) (width 0.4064) (layer "F.Cu") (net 4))
 (segment (start 143.51 103.632) (end 143.51 107.696) (width 0.4064) (layer "F.Cu") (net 4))
 (segment (start 144.285 102.857) (end 143.51 103.632) (width 0.4064) (layer "F.Cu") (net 4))
 (segment (start 154.347 101.981) (end 152.335 101.981) (width 0.4064) (layer "F.Cu") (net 4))
 (segment (start 151.192 100.838) (end 152.335 101.981) (width 0.4064) (layer "F.Cu") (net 4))
 (segment (start 144.526 101.854) (end 145.542 100.838) (width 0.4064) (layer "F.Cu") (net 4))
 (segment (start 145.542 100.838) (end 151.192 100.838) (width 0.4064) (layer "F.Cu") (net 4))
 (segment (start 146.05 110.236) (end 147.6325 110.236) (width 0.4064) (layer "F.Cu") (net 4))
 (segment (start 144.526 102.857) (end 144.526 101.854) (width 0.4064) (layer "F.Cu") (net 4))
 (segment (start 152.0875 107.3835) (end 152.0875 110.236) (width 0.4064) (layer "F.Cu") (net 3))
 (segment (start 154.41592 112.56442) (end 154.41592 118.63408) (width 0.4064) (layer "F.Cu") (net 3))
 (segment (start 151.21 122.747) (end 152.415 123.952) (width 0.4064) (layer "F.Cu") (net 3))
 (segment (start 154.41592 118.63408) (end 152.654 120.396) (width 0.4064) (layer "F.Cu") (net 3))
 (segment (start 152.415 123.952) (end 155.146 121.221) (width 0.4064) (layer "F.Cu") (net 3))
 (segment (start 150.495 105.791) (end 152.0875 107.3835) (width 0.4064) (layer "F.Cu") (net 3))
 (segment (start 151.21 120.396) (end 151.21 122.747) (width 0.4064) (layer "F.Cu") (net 3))
 (segment (start 155.146 121.221) (end 155.448 121.221) (width 0.4064) (layer "F.Cu") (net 3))
 (segment (start 152.654 120.396) (end 151.21 120.396) (width 0.4064) (layer "F.Cu") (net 3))
 (segment (start 152.0875 110.236) (end 154.41592 112.56442) (width 0.4064) (layer "F.Cu") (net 3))
 (segment (start 147.385 105.791) (end 150.495 105.791) (width 0.4064) (layer "F.Cu") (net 3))
 (segment (start 155.448 117.1195) (end 155.448 119.571) (width 0.4064) (layer "F.Cu") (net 5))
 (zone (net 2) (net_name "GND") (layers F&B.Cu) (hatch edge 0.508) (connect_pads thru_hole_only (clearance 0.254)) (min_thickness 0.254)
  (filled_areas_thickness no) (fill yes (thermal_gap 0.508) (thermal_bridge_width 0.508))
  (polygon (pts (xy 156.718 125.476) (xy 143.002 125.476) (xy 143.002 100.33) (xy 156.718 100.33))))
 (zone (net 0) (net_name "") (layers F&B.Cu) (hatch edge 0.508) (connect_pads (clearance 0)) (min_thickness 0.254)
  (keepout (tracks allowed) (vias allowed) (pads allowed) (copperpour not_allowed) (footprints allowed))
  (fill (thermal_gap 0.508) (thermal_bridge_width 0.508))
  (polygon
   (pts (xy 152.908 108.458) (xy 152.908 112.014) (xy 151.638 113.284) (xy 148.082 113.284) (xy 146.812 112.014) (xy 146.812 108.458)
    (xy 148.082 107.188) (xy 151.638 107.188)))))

